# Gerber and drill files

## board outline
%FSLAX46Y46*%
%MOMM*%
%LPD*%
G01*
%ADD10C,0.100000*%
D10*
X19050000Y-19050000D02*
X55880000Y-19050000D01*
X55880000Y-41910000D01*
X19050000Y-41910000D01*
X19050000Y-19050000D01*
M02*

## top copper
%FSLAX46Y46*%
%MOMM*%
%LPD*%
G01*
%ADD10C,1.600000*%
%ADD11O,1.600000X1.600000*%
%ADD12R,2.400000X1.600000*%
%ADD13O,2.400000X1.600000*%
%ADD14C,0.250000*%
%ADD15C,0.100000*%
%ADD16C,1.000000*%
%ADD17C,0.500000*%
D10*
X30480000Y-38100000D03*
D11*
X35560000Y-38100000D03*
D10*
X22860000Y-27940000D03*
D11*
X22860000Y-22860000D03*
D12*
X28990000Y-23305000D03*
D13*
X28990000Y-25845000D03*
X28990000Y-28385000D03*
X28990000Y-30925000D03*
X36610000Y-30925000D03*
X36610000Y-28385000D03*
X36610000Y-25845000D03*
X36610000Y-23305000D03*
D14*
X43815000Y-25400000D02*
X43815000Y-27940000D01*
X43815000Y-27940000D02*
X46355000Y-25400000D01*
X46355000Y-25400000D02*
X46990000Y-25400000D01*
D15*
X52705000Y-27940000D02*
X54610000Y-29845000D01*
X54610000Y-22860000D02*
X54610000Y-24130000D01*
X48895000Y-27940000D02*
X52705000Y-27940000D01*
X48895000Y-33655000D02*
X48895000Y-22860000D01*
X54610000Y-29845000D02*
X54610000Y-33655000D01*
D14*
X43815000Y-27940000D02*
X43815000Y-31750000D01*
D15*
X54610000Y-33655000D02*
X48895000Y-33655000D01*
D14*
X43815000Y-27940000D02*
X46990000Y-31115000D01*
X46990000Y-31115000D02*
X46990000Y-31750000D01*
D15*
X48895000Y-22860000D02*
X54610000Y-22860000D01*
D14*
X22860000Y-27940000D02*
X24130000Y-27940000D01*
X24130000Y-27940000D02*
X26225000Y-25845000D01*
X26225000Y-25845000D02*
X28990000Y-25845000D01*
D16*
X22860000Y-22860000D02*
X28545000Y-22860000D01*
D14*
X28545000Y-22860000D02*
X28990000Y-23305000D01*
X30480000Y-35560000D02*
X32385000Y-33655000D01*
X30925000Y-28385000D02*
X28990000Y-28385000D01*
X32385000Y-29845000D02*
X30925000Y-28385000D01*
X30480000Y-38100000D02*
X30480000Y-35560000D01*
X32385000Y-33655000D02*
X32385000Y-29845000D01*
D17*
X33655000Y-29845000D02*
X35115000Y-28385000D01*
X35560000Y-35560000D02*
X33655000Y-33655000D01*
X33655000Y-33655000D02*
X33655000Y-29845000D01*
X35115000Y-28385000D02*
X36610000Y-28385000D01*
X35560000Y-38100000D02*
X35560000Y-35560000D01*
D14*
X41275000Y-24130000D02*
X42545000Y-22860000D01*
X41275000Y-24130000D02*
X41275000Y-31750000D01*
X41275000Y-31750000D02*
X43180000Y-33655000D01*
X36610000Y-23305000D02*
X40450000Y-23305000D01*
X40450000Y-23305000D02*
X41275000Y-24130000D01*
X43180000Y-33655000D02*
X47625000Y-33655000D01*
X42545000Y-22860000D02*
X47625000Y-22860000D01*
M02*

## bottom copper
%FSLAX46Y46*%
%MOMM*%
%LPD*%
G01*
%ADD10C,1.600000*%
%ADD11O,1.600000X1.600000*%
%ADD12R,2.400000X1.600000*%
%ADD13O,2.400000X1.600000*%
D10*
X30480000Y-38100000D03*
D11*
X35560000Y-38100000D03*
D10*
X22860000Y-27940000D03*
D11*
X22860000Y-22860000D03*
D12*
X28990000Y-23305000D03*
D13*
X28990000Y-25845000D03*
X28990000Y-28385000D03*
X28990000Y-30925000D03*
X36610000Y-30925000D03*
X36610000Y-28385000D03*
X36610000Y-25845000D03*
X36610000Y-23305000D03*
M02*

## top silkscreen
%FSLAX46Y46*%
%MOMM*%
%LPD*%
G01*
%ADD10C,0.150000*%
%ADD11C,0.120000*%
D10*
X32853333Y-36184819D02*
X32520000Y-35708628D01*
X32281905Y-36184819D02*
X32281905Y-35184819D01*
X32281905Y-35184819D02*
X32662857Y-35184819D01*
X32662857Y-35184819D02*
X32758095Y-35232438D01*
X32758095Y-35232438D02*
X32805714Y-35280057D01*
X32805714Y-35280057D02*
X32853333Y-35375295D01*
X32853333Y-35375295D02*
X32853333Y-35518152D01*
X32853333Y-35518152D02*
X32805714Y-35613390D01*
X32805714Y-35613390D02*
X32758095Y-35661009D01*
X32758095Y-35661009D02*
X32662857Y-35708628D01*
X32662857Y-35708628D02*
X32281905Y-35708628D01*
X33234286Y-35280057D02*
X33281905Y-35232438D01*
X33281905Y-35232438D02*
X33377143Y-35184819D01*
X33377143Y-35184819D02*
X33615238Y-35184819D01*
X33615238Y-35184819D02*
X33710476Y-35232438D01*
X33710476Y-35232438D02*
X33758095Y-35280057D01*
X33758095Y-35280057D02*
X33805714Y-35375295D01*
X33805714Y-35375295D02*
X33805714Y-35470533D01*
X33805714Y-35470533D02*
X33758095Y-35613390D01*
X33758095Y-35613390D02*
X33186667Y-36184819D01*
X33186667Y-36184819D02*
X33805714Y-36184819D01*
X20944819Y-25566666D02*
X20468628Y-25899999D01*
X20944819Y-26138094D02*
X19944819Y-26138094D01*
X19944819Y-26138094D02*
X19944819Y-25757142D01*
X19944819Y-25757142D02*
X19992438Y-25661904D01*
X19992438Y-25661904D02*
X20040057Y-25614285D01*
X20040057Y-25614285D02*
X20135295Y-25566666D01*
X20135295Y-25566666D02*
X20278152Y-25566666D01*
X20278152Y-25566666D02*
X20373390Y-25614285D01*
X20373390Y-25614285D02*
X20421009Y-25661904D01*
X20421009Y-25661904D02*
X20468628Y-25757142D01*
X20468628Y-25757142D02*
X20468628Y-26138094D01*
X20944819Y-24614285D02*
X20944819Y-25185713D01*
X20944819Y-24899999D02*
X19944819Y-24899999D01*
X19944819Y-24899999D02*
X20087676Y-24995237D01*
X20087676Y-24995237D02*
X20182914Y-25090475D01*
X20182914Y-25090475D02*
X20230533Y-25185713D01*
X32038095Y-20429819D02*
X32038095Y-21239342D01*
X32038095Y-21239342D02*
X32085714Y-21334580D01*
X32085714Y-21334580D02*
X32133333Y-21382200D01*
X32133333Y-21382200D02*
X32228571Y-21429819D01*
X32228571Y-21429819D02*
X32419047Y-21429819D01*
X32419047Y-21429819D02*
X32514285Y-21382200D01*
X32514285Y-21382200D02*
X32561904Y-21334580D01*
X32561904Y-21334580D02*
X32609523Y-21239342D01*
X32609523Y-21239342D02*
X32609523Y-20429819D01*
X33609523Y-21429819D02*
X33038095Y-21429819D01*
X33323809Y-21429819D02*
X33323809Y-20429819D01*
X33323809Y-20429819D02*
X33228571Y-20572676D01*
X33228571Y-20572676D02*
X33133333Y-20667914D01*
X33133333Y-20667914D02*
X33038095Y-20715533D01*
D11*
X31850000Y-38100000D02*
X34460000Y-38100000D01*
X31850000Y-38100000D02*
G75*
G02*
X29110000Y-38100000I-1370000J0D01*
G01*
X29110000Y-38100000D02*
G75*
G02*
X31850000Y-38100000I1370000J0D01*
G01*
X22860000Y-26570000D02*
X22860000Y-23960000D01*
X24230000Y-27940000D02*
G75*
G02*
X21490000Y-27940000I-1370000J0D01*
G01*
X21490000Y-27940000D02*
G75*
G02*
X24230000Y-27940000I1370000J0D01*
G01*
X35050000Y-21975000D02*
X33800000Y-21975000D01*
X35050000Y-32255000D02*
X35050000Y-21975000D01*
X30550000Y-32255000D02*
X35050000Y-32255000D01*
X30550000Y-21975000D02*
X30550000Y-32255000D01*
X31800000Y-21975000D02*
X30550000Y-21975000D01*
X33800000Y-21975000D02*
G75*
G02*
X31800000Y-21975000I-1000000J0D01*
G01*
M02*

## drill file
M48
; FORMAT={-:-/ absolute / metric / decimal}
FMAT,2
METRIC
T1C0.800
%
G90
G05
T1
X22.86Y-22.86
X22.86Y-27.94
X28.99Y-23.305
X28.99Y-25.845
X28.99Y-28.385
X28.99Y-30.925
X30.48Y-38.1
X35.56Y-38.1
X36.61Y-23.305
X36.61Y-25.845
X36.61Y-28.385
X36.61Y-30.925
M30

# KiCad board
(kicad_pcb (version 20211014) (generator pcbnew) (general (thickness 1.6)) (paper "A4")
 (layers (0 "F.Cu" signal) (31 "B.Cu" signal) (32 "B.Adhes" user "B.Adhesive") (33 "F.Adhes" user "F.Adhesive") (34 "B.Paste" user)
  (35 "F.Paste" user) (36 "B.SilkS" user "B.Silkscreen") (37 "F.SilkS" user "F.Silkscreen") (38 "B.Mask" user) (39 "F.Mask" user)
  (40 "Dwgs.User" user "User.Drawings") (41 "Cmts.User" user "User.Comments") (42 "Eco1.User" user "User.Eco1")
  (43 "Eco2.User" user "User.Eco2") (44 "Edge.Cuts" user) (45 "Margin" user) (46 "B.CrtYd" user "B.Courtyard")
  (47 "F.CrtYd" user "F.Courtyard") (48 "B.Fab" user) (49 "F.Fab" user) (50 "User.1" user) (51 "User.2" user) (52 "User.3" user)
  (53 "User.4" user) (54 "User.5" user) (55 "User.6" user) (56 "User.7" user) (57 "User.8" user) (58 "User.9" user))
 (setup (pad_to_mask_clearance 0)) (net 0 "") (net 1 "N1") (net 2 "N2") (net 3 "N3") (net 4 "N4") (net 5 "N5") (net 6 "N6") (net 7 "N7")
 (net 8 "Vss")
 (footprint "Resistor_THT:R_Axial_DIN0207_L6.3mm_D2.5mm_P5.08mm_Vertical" (layer "F.Cu") (at 30.48 38.1)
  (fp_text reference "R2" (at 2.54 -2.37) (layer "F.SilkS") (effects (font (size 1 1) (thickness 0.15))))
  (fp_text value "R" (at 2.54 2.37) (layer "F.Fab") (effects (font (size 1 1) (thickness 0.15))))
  (fp_line (start 1.37 0) (end 3.98 0) (layer "F.SilkS") (width 0.12))
  (fp_circle (center 0 0) (end 1.37 0) (layer "F.SilkS") (width 0.12) (fill none))
  (pad "1" thru_hole circle (at 0 0) (size 1.6 1.6) (drill 0.8) (layers *.Cu *.Mask) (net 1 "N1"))
  (pad "2" thru_hole oval (at 5.08 0) (size 1.6 1.6) (drill 0.8) (layers *.Cu *.Mask) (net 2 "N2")))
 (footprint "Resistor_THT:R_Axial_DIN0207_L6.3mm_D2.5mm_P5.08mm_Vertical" (layer "F.Cu") (at 22.86 27.94 90)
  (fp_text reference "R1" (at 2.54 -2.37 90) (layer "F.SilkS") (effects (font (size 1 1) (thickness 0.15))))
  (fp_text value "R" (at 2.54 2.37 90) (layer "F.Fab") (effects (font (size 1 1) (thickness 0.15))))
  (fp_line (start 1.37 0) (end 3.98 0) (layer "F.SilkS") (width 0.12))
  (fp_circle (center 0 0) (end 1.37 0) (layer "F.SilkS") (width 0.12) (fill none))
  (pad "1" thru_hole circle (at 0 0 90) (size 1.6 1.6) (drill 0.8) (layers *.Cu *.Mask) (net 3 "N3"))
  (pad "2" thru_hole oval (at 5.08 0 90) (size 1.6 1.6) (drill 0.8) (layers *.Cu *.Mask) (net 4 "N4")))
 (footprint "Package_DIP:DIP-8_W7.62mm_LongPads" (layer "F.Cu") (at 28.99 23.305)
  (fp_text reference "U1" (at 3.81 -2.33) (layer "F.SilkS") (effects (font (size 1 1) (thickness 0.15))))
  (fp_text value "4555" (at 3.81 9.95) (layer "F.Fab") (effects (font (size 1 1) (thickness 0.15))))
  (fp_line (start 6.06 -1.33) (end 4.81 -1.33) (layer "F.SilkS") (width 0.12))
  (fp_line (start 6.06 8.95) (end 6.06 -1.33) (layer "F.SilkS") (width 0.12))
  (fp_line (start 1.56 8.95) (end 6.06 8.95) (layer "F.SilkS") (width 0.12))
  (fp_line (start 1.56 -1.33) (end 1.56 8.95) (layer "F.SilkS") (width 0.12))
  (fp_line (start 2.81 -1.33) (end 1.56 -1.33) (layer "F.SilkS") (width 0.12))
  (fp_arc (start 4.81 -1.33) (mid 3.81 -0.33) (end 2.81 -1.33) (layer "F.SilkS") (width 0.12))
  (pad "1" thru_hole rect (at 0 0) (size 2.4 1.6) (drill 0.8) (layers *.Cu *.Mask) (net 4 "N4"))
  (pad "2" thru_hole oval (at 0 2.54) (size 2.4 1.6) (drill 0.8) (layers *.Cu *.Mask) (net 3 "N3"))
  (pad "3" thru_hole oval (at 0 5.08) (size 2.4 1.6) (drill 0.8) (layers *.Cu *.Mask) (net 1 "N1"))
  (pad "4" thru_hole oval (at 0 7.62) (size 2.4 1.6) (drill 0.8) (layers *.Cu *.Mask) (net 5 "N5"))
  (pad "5" thru_hole oval (at 7.62 7.62) (size 2.4 1.6) (drill 0.8) (layers *.Cu *.Mask) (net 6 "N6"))
  (pad "6" thru_hole oval (at 7.62 5.08) (size 2.4 1.6) (drill 0.8) (layers *.Cu *.Mask) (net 2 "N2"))
  (pad "7" thru_hole oval (at 7.62 2.54) (size 2.4 1.6) (drill 0.8) (layers *.Cu *.Mask) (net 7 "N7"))
  (pad "8" thru_hole oval (at 7.62 0) (size 2.4 1.6) (drill 0.8) (layers *.Cu *.Mask) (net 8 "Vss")))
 (gr_rect (start 19.05 19.05) (end 55.88 41.91) (layer "Edge.Cuts") (width 0.1) (fill none))
 (segment (start 43.815 25.4) (end 43.815 27.94) (width 0.25) (layer "F.Cu") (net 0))
 (segment (start 43.815 27.94) (end 46.355 25.4) (width 0.25) (layer "F.Cu") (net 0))
 (segment (start 46.355 25.4) (end 46.99 25.4) (width 0.25) (layer "F.Cu") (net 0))
 (segment (start 52.705 27.94) (end 54.61 29.845) (width 0.1) (layer "F.Cu") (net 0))
 (segment (start 54.61 22.86) (end 54.61 24.13) (width 0.1) (layer "F.Cu") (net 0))
 (segment (start 48.895 27.94) (end 52.705 27.94) (width 0.1) (layer "F.Cu") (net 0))
 (segment (start 48.895 33.655) (end 48.895 22.86) (width 0.1) (layer "F.Cu") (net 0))
 (segment (start 54.61 29.845) (end 54.61 33.655) (width 0.1) (layer "F.Cu") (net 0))
 (segment (start 43.815 27.94) (end 43.815 31.75) (width 0.25) (layer "F.Cu") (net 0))
 (segment (start 54.61 33.655) (end 48.895 33.655) (width 0.1) (layer "F.Cu") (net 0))
 (segment (start 43.815 27.94) (end 46.99 31.115) (width 0.25) (layer "F.Cu") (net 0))
 (segment (start 46.99 31.115) (end 46.99 31.75) (width 0.25) (layer "F.Cu") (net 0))
 (segment (start 48.895 22.86) (end 54.61 22.86) (width 0.1) (layer "F.Cu") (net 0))
 (segment (start 22.86 27.94) (end 24.13 27.94) (width 0.25) (layer "F.Cu") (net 3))
 (segment (start 24.13 27.94) (end 26.225 25.845) (width 0.25) (layer "F.Cu") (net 3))
 (segment (start 26.225 25.845) (end 28.99 25.845) (width 0.25) (layer "F.Cu") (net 3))
 (segment (start 22.86 22.86) (end 28.545 22.86) (width 1) (layer "F.Cu") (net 4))
 (segment (start 28.545 22.86) (end 28.99 23.305) (width 0.25) (layer "F.Cu") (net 4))
 (segment (start 30.48 35.56) (end 32.385 33.655) (width 0.25) (layer "F.Cu") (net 1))
 (segment (start 30.925 28.385) (end 28.99 28.385) (width 0.25) (layer "F.Cu") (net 1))
 (segment (start 32.385 29.845) (end 30.925 28.385) (width 0.25) (layer "F.Cu") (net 1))
 (segment (start 30.48 38.1) (end 30.48 35.56) (width 0.25) (layer "F.Cu") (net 1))
 (segment (start 32.385 33.655) (end 32.385 29.845) (width 0.25) (layer "F.Cu") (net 1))
 (segment (start 33.655 29.845) (end 35.115 28.385) (width 0.5) (layer "F.Cu") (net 2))
 (segment (start 35.56 35.56) (end 33.655 33.655) (width 0.5) (layer "F.Cu") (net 2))
 (segment (start 33.655 33.655) (end 33.655 29.845) (width 0.5) (layer "F.Cu") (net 2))
 (segment (start 35.115 28.385) (end 36.61 28.385) (width 0.5) (layer "F.Cu") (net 2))
 (segment (start 35.56 38.1) (end 35.56 35.56) (width 0.5) (layer "F.Cu") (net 2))
 (segment (start 41.275 24.13) (end 42.545 22.86) (width 0.25) (layer "F.Cu") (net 8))
 (segment (start 41.275 24.13) (end 41.275 31.75) (width 0.25) (layer "F.Cu") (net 8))
 (segment (start 41.275 31.75) (end 43.18 33.655) (width 0.25) (layer "F.Cu") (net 8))
 (segment (start 36.61 23.305) (end 40.45 23.305) (width 0.25) (layer "F.Cu") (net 8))
 (segment (start 40.45 23.305) (end 41.275 24.13) (width 0.25) (layer "F.Cu") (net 8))
 (segment (start 43.18 33.655) (end 47.625 33.655) (width 0.25) (layer "F.Cu") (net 8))
 (segment (start 42.545 22.86) (end 47.625 22.86) (width 0.25) (layer "F.Cu") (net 8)))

